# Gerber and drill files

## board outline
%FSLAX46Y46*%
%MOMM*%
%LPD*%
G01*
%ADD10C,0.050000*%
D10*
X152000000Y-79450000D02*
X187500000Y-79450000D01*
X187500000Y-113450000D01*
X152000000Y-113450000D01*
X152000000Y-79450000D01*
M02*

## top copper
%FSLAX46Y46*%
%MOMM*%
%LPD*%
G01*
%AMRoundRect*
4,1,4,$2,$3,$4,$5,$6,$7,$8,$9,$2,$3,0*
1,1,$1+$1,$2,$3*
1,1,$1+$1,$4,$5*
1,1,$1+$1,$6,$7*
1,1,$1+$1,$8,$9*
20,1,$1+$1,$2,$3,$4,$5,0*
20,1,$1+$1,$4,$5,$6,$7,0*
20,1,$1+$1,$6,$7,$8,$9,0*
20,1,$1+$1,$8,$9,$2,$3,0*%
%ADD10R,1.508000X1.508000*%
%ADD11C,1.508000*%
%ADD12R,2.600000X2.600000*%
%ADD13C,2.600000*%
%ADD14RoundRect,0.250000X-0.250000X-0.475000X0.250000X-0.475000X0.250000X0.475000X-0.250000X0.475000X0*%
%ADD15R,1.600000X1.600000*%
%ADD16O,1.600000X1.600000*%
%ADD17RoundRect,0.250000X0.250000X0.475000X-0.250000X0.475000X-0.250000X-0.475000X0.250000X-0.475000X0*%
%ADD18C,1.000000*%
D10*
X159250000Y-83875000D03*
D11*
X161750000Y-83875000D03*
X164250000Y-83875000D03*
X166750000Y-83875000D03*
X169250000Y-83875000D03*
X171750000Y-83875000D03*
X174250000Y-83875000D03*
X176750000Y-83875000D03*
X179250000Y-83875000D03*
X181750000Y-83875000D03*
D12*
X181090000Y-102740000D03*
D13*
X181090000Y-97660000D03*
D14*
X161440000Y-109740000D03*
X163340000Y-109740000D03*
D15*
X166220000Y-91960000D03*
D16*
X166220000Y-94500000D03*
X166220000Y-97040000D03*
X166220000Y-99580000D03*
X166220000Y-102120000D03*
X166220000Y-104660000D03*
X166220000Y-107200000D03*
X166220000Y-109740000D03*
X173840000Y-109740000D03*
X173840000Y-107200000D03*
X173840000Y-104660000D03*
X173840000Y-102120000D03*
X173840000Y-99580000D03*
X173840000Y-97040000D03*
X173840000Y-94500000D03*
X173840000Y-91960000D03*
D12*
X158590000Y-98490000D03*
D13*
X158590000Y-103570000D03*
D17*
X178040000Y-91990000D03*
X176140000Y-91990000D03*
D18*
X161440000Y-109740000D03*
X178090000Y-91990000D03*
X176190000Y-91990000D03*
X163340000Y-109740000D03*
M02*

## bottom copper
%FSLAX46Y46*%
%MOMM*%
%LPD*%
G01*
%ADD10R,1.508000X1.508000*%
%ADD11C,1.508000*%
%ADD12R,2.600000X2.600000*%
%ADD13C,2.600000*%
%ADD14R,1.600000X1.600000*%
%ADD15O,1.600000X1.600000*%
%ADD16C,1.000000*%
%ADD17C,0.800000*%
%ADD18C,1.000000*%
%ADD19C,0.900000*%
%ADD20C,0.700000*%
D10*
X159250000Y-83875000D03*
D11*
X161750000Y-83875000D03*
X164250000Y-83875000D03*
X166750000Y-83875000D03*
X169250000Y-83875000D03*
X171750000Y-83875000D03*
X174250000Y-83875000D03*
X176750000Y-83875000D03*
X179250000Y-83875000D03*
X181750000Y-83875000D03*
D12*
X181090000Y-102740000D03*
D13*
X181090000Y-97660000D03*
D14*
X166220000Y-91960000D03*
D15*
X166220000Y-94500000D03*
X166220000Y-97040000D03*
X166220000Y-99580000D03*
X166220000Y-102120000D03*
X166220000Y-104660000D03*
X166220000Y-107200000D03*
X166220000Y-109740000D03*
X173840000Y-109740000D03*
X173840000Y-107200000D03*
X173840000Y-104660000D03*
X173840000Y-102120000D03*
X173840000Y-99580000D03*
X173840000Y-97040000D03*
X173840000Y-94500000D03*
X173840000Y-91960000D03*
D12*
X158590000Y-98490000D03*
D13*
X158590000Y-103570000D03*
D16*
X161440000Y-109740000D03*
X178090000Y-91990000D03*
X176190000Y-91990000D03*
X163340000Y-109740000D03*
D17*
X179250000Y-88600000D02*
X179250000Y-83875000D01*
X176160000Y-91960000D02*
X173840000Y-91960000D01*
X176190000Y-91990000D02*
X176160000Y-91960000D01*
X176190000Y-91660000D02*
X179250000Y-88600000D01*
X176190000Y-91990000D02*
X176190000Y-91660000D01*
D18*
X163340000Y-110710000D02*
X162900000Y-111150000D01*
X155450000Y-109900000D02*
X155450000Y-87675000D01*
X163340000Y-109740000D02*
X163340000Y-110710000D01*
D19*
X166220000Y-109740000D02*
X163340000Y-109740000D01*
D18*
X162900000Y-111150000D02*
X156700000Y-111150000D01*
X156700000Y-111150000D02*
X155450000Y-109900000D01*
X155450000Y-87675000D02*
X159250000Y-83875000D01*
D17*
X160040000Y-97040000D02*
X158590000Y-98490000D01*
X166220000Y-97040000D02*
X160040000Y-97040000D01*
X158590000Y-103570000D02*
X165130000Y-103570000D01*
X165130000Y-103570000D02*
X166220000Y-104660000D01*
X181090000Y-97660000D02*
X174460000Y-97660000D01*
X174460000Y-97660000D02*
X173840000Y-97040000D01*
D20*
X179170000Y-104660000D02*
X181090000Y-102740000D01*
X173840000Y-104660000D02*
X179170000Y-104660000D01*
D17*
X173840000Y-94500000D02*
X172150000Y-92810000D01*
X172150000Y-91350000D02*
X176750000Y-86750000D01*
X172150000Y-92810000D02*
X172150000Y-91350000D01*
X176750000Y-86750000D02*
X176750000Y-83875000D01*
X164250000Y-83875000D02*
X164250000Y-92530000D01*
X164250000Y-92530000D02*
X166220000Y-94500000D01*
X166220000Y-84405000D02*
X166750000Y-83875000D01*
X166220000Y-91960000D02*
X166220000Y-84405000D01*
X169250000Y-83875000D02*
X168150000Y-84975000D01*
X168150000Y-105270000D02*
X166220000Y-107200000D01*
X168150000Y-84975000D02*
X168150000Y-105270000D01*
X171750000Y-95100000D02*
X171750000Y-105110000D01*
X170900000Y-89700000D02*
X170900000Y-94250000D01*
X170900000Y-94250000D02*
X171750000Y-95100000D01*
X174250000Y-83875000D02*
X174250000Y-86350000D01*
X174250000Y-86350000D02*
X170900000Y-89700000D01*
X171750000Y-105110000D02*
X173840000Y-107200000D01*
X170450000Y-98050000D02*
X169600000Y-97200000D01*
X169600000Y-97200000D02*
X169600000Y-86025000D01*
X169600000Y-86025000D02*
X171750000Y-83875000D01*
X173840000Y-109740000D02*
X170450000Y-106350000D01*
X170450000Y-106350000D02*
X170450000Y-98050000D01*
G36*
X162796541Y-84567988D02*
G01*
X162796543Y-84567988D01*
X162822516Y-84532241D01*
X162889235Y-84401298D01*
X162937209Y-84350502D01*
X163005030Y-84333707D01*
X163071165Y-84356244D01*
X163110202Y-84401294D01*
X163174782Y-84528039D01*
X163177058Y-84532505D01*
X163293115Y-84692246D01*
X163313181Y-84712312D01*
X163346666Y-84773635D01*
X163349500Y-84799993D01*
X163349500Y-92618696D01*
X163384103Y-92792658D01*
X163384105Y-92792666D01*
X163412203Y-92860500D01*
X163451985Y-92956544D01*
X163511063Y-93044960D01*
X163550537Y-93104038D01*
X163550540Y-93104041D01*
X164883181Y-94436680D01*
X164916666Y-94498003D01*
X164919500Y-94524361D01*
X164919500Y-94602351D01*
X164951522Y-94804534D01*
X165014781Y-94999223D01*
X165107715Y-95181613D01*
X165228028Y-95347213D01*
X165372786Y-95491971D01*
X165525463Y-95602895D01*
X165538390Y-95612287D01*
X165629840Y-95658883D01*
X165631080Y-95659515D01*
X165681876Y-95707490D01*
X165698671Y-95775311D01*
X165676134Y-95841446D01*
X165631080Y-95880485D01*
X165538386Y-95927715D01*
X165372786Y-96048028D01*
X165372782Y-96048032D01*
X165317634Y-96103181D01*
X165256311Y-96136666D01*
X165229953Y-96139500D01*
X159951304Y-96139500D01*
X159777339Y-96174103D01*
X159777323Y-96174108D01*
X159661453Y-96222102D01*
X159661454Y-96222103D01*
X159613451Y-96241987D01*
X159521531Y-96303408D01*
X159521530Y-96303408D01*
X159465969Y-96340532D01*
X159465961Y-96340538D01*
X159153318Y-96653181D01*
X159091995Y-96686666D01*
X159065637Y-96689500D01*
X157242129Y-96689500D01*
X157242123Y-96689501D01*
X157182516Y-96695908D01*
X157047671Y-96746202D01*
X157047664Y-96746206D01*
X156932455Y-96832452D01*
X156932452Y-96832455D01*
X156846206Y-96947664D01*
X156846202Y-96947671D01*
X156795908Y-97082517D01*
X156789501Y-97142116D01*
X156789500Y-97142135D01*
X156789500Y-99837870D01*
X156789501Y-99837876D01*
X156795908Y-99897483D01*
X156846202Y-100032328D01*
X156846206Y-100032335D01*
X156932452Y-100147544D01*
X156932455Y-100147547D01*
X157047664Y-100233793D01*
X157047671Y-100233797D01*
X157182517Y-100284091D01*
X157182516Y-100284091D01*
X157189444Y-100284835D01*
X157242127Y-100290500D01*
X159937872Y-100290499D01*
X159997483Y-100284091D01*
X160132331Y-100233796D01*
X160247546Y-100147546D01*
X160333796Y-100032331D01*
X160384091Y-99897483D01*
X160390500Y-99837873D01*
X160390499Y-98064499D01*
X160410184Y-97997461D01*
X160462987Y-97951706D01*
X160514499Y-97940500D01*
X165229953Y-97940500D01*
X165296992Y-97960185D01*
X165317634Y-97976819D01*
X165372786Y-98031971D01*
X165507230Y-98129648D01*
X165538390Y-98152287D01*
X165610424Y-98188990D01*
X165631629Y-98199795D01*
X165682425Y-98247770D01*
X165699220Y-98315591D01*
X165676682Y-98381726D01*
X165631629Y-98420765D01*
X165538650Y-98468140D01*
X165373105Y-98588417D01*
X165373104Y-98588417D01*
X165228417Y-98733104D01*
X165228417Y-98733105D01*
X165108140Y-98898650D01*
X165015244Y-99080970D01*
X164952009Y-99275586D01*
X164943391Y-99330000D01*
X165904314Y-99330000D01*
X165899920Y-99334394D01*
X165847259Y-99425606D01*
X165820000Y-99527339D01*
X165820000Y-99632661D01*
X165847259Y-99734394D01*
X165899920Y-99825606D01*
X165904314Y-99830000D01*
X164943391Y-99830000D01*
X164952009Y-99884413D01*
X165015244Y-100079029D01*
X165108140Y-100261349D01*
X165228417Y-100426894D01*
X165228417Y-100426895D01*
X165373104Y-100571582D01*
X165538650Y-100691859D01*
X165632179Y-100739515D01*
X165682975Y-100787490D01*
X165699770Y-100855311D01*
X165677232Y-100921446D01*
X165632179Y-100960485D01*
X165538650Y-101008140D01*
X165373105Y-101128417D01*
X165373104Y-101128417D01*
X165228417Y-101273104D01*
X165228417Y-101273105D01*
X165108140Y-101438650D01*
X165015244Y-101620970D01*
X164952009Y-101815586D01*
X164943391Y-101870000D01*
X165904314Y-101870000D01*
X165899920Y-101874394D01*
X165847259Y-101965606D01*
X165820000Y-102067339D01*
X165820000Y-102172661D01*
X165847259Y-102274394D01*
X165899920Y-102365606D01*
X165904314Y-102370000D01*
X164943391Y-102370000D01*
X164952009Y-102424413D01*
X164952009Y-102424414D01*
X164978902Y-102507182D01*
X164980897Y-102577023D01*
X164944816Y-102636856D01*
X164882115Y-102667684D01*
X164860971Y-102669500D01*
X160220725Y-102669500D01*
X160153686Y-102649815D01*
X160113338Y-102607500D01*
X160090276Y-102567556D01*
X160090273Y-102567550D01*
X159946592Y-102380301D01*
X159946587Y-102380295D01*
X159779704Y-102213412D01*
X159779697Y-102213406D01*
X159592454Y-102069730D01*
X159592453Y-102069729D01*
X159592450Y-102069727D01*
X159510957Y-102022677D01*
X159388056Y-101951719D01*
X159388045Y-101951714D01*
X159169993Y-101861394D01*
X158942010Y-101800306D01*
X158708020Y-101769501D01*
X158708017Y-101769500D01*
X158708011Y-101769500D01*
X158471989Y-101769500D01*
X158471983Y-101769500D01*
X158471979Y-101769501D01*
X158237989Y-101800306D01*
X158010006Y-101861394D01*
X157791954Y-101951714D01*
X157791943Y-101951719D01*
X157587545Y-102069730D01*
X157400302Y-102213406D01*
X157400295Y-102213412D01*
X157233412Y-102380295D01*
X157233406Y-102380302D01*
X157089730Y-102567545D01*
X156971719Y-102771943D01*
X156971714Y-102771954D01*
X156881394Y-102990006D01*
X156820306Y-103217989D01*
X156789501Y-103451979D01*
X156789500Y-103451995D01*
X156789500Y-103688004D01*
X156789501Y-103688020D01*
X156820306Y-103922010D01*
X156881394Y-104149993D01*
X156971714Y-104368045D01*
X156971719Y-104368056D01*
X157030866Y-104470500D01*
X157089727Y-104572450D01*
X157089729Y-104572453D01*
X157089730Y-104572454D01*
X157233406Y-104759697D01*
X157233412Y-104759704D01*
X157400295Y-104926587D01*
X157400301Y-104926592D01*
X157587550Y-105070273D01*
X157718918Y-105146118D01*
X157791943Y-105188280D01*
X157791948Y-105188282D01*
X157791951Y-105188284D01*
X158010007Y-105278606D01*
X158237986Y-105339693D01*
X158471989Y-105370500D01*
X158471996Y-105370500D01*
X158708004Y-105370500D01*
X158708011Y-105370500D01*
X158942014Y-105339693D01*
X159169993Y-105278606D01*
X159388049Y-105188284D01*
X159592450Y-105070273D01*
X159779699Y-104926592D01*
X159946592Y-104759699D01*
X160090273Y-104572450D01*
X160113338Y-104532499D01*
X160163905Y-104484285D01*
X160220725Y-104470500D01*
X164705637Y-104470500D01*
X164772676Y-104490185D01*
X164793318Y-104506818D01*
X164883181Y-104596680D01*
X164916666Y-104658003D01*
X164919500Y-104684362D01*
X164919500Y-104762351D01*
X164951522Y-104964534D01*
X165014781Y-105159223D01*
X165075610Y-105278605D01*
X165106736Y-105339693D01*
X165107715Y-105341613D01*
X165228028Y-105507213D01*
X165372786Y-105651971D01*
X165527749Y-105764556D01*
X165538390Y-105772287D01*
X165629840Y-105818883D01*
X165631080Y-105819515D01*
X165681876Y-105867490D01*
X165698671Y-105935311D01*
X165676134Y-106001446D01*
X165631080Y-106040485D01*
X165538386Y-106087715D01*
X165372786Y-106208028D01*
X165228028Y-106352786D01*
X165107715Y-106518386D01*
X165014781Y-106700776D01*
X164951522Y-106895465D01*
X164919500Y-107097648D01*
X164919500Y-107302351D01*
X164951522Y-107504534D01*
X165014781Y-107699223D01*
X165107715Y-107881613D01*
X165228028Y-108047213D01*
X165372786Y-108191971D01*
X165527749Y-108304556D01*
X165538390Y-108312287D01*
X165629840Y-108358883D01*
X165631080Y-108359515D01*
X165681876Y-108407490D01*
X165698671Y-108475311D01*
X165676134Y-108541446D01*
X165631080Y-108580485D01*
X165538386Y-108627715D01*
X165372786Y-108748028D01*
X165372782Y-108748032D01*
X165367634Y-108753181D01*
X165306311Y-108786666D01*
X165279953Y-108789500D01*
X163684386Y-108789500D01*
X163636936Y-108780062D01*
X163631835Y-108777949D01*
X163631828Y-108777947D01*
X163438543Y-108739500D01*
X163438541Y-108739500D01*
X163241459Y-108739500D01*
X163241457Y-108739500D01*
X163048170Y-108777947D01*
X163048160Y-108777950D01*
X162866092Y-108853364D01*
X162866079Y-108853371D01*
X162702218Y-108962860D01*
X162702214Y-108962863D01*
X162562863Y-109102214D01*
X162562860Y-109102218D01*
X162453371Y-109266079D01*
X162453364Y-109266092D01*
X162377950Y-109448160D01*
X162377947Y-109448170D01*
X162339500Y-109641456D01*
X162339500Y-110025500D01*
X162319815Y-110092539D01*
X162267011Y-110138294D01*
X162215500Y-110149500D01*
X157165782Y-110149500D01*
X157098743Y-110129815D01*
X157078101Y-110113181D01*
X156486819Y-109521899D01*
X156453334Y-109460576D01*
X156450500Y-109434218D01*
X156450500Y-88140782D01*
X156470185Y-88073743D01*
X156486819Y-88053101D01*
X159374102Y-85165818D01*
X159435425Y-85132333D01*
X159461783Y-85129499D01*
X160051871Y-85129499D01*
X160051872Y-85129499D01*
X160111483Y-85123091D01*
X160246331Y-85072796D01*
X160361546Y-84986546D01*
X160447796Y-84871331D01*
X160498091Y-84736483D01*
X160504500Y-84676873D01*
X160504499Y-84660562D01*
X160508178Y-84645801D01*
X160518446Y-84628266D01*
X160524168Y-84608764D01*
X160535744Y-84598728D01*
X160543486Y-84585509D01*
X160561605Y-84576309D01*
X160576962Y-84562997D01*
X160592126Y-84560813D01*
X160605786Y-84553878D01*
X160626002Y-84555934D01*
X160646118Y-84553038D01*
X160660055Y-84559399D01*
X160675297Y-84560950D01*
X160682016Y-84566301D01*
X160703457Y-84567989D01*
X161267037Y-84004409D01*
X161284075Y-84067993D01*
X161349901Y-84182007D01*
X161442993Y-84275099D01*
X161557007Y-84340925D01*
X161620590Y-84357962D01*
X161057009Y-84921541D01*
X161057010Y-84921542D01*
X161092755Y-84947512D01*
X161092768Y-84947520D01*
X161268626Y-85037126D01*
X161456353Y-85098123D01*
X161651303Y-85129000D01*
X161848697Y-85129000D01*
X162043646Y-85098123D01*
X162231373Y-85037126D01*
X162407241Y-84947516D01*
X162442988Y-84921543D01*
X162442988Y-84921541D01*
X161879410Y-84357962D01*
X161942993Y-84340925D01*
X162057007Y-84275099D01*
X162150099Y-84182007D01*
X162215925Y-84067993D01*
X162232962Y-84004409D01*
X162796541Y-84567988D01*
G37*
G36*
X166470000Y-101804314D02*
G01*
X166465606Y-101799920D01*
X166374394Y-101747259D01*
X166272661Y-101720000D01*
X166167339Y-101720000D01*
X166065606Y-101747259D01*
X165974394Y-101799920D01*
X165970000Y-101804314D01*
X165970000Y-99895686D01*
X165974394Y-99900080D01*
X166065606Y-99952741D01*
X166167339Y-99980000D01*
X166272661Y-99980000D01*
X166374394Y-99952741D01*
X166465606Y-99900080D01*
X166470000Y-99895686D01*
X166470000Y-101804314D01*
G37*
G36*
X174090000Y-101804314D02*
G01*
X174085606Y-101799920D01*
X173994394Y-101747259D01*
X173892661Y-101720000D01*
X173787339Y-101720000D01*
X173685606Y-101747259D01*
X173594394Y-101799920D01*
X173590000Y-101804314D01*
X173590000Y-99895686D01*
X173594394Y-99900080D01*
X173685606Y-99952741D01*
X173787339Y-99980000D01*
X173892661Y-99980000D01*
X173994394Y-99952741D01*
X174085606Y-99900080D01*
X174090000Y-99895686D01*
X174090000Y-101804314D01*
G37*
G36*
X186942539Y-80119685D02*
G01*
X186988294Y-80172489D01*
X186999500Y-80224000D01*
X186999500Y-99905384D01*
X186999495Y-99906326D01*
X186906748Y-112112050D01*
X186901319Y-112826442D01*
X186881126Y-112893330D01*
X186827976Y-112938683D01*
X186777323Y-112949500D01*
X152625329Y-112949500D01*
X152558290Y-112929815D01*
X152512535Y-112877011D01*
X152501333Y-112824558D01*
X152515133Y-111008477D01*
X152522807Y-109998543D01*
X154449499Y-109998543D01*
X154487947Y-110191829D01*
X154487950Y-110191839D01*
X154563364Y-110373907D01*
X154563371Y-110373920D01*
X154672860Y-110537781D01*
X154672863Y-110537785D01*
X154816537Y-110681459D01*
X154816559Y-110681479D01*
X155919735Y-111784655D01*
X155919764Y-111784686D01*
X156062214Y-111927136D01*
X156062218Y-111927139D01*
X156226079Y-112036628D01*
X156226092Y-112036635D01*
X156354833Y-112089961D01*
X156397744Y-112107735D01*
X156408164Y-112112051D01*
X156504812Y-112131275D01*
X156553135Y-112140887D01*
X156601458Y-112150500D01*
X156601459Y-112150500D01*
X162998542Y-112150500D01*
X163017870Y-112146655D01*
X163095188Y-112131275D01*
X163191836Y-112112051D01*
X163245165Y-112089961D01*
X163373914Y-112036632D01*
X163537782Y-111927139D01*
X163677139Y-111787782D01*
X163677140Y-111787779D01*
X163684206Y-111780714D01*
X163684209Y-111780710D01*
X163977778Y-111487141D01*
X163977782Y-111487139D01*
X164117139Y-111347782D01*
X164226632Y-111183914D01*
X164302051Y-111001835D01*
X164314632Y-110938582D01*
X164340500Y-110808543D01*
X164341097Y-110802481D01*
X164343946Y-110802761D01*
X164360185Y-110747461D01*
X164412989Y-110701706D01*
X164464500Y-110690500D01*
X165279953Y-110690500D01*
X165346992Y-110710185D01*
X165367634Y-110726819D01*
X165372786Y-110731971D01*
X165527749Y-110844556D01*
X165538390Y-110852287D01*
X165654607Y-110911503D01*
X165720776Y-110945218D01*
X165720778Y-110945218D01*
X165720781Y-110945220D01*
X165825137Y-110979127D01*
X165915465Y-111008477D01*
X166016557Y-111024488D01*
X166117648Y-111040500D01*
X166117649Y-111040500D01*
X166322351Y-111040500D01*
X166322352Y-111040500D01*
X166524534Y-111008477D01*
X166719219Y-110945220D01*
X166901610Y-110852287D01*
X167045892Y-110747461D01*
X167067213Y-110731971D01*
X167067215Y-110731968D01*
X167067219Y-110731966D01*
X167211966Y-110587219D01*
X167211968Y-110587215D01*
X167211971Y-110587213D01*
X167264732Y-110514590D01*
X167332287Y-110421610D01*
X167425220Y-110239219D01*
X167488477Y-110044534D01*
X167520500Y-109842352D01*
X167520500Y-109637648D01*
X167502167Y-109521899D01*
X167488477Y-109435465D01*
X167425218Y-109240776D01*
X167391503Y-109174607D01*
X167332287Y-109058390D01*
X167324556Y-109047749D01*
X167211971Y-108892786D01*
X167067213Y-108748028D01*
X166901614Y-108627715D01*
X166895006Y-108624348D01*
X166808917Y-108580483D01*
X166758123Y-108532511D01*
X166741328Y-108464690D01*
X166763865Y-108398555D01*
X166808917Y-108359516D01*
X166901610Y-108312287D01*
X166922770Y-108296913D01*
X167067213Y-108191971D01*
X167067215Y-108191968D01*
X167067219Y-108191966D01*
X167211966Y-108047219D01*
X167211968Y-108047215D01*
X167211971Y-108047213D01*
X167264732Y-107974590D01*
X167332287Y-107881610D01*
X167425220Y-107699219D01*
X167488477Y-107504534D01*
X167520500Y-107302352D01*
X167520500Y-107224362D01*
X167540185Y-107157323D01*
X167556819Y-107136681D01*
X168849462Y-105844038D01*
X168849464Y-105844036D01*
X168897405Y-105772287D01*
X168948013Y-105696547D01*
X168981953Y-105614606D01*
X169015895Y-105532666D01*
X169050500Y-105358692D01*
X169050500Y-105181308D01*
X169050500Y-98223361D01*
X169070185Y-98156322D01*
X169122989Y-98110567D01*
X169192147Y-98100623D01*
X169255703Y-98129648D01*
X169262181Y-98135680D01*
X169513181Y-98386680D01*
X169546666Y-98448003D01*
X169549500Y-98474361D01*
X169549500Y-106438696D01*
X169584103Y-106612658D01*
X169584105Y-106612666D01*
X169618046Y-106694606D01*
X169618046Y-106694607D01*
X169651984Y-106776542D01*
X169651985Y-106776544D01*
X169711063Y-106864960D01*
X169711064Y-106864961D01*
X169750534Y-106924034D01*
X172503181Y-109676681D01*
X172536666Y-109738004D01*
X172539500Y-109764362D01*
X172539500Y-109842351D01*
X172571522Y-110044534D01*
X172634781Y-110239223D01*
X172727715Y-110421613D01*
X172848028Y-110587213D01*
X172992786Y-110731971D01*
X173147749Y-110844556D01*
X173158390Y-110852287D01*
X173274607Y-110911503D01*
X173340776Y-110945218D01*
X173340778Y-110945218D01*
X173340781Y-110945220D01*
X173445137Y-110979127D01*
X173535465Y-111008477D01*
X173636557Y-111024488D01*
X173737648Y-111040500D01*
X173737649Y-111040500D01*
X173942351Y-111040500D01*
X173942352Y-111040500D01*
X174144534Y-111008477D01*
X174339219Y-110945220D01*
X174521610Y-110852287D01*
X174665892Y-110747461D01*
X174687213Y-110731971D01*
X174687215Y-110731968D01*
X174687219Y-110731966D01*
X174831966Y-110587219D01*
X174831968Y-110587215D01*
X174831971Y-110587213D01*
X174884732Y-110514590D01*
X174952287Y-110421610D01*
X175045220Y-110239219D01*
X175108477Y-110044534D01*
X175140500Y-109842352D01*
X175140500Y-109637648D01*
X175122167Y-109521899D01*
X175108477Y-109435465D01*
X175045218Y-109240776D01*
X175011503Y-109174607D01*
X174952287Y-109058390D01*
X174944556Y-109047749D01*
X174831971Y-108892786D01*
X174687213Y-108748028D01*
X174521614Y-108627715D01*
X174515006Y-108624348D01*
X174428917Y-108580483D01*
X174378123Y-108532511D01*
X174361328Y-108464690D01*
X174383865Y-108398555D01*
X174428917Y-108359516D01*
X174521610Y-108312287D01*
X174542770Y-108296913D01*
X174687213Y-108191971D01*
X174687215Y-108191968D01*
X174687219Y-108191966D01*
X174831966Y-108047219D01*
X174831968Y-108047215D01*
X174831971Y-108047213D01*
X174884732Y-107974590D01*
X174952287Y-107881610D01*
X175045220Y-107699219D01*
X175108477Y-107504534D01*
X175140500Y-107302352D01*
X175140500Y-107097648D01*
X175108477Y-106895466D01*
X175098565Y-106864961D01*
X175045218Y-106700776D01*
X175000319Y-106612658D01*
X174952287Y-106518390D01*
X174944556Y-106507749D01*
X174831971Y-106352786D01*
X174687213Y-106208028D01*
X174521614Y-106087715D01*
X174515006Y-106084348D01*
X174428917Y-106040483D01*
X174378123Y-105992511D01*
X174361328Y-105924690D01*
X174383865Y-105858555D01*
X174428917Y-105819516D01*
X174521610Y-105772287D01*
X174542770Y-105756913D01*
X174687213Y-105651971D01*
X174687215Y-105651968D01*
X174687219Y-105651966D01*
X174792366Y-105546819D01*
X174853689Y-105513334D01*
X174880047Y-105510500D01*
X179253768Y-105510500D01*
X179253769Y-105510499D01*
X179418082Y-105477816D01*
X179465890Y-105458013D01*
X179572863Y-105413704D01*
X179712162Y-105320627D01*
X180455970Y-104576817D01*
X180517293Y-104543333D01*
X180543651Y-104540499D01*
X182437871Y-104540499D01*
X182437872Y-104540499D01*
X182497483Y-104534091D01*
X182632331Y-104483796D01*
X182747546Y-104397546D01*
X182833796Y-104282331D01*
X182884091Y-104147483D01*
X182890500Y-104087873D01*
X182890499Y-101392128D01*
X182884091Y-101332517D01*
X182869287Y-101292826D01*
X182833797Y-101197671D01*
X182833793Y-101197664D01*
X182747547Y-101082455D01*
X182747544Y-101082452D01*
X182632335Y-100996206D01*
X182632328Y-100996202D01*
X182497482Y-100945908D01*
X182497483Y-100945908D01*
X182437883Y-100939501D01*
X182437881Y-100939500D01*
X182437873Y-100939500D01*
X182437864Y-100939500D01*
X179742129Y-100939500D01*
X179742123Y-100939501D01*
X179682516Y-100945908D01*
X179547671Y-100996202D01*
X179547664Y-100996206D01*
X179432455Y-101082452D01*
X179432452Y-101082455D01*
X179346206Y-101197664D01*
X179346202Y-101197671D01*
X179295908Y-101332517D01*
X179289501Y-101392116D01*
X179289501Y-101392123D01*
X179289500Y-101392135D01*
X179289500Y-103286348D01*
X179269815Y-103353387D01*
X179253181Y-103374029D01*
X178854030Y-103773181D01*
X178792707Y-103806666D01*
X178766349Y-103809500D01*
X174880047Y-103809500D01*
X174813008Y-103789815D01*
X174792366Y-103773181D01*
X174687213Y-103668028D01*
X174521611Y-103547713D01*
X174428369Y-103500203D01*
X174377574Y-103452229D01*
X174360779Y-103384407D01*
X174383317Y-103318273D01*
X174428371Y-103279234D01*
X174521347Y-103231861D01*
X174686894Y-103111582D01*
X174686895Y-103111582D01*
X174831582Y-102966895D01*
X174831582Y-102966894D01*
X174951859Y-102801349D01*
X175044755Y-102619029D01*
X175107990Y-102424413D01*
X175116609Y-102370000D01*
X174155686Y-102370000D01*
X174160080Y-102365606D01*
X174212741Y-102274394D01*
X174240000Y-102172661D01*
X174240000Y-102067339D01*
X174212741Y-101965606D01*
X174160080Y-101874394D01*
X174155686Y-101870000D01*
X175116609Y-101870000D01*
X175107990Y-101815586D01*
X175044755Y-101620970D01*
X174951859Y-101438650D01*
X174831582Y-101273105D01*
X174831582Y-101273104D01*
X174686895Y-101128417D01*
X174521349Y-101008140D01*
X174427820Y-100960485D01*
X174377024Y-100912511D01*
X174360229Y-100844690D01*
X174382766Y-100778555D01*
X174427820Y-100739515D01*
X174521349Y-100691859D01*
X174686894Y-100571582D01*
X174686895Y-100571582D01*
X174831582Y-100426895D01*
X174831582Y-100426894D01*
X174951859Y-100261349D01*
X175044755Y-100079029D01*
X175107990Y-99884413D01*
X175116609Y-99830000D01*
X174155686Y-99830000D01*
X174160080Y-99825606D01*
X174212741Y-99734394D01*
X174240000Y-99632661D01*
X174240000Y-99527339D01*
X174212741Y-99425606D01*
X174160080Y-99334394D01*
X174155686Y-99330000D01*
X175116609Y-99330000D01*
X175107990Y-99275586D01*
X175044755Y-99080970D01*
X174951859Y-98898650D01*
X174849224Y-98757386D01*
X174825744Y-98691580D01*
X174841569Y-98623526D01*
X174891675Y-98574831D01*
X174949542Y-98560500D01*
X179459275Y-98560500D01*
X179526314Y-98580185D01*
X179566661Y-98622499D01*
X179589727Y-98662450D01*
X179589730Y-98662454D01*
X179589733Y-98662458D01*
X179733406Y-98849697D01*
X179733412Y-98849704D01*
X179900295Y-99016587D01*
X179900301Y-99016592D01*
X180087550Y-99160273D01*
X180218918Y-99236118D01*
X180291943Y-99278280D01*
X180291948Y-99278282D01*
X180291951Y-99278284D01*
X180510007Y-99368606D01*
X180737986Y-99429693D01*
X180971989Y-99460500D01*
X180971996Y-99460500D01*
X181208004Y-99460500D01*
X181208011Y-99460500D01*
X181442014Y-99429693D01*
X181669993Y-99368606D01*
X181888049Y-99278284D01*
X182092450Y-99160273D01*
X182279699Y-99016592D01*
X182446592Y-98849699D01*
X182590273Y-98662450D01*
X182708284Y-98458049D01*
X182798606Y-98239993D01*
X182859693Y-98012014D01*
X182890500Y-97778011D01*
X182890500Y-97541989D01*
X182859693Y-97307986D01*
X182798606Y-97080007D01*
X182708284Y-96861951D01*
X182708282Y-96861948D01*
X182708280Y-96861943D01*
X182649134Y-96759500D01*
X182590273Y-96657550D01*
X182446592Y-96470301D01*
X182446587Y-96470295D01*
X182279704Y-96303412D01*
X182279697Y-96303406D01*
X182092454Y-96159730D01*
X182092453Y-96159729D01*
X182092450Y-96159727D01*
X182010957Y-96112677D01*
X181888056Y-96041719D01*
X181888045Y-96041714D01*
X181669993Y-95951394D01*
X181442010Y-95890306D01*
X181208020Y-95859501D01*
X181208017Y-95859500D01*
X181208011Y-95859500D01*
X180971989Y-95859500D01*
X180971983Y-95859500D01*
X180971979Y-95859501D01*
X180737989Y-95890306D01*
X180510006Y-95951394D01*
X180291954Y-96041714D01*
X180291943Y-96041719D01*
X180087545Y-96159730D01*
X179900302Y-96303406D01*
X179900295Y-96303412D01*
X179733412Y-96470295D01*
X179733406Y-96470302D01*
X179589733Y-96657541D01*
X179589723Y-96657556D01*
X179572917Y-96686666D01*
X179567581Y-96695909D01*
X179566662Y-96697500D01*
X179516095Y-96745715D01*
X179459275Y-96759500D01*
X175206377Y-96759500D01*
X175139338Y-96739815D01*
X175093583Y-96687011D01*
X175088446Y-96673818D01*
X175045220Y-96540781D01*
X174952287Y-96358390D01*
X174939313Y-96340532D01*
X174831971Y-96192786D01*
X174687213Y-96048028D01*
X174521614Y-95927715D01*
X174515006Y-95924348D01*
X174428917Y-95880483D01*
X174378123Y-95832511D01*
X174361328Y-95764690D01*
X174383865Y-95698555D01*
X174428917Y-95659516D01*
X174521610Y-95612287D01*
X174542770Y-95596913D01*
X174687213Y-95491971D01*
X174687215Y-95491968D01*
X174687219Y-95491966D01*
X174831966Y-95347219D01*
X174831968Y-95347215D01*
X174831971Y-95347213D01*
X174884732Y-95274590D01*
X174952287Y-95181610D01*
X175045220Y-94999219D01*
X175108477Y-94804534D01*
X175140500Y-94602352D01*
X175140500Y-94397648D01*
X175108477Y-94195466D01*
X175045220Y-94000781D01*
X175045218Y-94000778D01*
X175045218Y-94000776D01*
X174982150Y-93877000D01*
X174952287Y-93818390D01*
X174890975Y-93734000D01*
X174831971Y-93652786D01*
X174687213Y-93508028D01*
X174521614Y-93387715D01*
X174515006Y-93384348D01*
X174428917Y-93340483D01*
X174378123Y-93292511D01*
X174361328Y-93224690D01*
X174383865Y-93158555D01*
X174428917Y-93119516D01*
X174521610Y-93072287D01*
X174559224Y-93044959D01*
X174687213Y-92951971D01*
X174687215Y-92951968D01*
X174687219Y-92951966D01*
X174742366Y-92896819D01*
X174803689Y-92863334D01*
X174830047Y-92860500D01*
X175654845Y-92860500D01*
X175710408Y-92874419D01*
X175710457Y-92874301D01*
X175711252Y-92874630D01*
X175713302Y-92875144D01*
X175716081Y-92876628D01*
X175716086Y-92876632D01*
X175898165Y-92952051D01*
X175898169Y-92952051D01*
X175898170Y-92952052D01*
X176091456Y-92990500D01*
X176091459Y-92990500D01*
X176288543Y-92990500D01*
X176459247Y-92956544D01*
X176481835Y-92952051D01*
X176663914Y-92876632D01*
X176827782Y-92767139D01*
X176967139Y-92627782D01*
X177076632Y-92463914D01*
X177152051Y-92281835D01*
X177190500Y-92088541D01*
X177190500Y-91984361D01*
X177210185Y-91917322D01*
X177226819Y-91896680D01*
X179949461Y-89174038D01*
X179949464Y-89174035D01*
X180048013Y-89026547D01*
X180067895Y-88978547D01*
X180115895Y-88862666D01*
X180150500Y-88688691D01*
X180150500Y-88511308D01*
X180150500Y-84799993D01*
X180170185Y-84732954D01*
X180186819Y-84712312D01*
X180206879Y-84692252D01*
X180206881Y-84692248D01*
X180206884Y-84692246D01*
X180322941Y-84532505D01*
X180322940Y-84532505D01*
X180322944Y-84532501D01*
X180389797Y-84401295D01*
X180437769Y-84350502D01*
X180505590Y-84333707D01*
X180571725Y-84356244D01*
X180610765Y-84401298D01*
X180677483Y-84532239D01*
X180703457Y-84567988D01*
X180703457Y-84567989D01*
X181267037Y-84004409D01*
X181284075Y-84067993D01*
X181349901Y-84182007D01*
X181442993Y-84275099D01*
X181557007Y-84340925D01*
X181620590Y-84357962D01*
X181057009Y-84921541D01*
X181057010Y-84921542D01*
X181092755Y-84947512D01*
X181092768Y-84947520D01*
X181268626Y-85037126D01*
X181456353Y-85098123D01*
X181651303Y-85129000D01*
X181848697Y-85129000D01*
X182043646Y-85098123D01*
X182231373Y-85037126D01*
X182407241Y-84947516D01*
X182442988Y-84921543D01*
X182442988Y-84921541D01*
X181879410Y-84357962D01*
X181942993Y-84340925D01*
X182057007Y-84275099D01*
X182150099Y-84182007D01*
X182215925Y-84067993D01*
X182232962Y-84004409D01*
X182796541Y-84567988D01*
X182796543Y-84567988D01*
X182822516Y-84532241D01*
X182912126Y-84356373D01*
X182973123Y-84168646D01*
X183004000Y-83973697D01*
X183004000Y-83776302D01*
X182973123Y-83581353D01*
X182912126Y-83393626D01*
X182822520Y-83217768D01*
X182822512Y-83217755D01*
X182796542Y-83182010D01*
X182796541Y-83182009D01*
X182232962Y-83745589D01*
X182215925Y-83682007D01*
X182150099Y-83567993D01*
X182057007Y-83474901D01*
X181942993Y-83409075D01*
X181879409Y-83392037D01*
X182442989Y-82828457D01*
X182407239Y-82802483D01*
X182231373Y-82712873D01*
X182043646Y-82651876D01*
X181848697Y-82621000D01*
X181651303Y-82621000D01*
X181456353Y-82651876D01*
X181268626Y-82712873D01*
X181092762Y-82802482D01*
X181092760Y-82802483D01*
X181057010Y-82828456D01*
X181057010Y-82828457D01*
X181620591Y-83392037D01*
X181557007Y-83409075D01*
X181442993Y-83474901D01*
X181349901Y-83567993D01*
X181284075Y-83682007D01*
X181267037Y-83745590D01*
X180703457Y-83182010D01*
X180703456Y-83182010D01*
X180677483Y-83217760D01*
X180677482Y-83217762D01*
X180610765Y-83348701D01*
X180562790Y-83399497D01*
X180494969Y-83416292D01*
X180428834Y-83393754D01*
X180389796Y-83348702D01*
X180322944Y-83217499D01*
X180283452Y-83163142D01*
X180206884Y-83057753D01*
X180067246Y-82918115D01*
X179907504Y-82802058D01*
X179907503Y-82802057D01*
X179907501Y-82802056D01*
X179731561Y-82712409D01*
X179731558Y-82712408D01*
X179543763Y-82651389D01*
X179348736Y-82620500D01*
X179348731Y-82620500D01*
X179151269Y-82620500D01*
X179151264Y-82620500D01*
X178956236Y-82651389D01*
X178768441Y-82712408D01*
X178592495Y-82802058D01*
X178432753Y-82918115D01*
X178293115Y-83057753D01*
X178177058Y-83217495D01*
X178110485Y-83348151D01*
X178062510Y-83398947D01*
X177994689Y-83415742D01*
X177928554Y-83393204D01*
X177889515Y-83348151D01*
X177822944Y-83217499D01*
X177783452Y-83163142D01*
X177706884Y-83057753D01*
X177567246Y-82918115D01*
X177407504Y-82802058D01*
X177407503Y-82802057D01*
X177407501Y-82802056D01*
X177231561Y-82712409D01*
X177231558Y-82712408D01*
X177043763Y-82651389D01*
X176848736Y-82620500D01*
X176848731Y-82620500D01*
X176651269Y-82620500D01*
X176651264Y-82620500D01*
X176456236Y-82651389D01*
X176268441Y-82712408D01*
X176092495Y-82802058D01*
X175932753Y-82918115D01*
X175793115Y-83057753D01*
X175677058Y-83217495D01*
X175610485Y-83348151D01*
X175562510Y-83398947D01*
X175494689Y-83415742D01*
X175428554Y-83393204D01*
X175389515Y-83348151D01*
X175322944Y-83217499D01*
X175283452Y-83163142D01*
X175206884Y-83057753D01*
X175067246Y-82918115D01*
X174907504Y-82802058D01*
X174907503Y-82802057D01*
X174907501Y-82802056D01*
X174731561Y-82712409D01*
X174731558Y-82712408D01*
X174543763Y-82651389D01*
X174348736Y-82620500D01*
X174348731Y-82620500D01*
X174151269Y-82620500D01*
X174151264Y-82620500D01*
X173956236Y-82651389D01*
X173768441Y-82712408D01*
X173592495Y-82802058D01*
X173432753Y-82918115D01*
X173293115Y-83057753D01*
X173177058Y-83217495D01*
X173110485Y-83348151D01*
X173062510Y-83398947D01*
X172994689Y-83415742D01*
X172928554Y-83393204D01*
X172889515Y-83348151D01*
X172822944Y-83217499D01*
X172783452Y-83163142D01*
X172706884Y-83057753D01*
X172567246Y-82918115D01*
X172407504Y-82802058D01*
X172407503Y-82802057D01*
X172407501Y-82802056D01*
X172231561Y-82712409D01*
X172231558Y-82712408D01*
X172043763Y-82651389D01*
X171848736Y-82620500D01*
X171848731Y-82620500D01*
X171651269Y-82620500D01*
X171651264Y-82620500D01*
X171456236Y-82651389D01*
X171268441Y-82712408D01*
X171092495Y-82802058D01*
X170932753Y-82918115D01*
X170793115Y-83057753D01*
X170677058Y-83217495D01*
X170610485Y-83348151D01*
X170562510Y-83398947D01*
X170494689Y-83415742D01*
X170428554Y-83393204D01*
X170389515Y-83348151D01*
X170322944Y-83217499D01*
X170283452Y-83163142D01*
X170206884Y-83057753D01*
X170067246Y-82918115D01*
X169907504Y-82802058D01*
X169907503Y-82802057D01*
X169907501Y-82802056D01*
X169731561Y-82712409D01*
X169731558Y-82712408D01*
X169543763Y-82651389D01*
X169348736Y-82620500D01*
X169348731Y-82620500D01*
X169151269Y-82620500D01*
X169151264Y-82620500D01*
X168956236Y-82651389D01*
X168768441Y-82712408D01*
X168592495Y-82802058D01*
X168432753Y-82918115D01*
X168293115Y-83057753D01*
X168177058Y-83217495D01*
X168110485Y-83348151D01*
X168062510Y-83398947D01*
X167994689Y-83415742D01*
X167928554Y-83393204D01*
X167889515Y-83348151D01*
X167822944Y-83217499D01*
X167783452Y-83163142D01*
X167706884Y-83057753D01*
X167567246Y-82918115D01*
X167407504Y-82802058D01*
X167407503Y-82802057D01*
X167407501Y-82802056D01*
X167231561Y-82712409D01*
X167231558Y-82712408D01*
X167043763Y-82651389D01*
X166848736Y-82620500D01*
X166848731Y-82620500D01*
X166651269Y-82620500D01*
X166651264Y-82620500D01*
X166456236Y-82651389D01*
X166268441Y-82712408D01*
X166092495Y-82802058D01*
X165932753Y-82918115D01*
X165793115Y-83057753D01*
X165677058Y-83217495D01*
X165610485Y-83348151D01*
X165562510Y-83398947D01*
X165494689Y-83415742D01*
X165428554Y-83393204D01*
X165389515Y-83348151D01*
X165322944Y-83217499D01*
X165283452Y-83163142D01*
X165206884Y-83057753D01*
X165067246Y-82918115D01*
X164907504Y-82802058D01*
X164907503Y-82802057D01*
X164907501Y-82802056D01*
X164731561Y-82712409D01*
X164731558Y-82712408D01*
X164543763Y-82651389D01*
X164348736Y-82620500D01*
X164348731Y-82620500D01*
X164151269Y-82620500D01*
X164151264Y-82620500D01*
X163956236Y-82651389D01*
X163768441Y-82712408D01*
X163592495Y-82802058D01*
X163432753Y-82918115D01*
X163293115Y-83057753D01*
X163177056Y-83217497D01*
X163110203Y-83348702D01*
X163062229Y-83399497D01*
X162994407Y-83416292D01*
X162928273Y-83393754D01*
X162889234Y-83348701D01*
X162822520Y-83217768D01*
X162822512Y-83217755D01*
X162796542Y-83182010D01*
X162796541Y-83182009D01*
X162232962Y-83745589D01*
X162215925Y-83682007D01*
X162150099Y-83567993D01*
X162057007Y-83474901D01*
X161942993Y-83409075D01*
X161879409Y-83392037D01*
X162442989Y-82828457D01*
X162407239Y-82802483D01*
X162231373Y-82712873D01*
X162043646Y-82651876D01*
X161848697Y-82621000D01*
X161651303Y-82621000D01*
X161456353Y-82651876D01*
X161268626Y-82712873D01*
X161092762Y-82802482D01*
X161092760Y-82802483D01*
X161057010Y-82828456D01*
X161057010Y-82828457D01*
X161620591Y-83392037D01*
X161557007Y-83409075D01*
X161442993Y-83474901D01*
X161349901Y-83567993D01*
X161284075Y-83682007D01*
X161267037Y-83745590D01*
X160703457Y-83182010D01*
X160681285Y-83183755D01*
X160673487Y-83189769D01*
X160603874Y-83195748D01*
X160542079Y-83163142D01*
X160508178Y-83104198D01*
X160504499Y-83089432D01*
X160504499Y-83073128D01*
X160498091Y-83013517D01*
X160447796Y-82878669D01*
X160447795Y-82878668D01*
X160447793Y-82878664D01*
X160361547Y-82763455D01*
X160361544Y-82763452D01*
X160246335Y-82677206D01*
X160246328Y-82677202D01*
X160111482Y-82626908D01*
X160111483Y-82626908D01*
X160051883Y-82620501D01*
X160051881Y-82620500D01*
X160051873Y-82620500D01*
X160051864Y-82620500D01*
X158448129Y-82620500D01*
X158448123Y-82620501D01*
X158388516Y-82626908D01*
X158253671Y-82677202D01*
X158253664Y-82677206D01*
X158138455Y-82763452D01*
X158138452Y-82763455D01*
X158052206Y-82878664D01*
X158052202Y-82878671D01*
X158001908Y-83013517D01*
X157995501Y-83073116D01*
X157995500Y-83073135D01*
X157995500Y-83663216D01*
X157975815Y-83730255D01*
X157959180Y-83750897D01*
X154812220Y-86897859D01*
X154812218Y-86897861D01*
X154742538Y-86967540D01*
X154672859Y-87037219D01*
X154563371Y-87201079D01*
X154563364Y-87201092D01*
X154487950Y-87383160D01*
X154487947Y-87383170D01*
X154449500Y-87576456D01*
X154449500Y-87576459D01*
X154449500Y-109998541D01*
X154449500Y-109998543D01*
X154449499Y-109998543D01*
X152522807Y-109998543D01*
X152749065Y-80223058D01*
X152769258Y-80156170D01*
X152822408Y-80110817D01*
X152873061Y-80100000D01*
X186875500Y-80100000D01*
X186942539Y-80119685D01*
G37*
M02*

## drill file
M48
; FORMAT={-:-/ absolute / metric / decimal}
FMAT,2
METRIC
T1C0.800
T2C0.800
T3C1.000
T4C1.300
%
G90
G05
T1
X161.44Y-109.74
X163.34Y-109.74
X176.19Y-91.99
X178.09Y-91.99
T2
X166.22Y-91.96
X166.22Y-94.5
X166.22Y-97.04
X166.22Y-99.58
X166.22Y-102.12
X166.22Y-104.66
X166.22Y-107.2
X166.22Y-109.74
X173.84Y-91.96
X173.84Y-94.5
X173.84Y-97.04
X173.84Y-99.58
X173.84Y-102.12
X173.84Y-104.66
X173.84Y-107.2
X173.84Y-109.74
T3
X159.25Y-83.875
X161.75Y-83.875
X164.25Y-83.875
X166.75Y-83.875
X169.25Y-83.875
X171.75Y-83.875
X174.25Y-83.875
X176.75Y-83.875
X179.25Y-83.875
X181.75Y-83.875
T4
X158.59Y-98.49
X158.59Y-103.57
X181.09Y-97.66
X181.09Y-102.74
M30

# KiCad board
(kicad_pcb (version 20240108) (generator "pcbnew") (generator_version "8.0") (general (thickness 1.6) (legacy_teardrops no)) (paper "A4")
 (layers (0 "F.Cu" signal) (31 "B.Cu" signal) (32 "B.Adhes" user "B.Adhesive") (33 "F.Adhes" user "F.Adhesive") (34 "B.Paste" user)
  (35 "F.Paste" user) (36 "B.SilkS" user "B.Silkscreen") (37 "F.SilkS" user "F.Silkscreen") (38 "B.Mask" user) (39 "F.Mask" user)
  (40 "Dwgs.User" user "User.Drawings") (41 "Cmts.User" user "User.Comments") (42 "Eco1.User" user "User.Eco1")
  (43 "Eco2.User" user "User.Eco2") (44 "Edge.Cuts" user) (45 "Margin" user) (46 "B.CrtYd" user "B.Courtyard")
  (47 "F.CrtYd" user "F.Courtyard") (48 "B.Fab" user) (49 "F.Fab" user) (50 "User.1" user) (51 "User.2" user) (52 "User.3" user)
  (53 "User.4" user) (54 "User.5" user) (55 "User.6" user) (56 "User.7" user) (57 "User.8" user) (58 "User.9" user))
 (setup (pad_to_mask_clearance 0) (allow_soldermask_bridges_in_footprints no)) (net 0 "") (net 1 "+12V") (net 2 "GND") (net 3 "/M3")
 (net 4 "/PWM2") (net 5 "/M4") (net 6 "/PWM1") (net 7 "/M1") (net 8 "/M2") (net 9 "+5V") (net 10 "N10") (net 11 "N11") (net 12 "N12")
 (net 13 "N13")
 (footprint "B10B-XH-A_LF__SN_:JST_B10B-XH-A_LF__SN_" (layer "F.Cu") (at 170.5 84.4 180)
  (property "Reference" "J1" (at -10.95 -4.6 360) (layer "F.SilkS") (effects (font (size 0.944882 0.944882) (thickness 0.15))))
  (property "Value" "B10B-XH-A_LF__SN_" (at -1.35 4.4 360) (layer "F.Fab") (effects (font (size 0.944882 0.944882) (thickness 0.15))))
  (pad "1" thru_hole rect (at 11.25 0.525 180) (size 1.508 1.508) (drill 1) (layers "*.Cu" "*.Mask") (remove_unused_layers no)
   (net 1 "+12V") (solder_mask_margin 0.102))
  (pad "2" thru_hole circle (at 8.75 0.525 180) (size 1.508 1.508) (drill 1) (layers "*.Cu" "*.Mask") (remove_unused_layers no)
   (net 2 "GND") (solder_mask_margin 0.102))
  (pad "3" thru_hole circle (at 6.25 0.525 180) (size 1.508 1.508) (drill 1) (layers "*.Cu" "*.Mask") (remove_unused_layers no)
   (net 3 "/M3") (solder_mask_margin 0.102))
  (pad "4" thru_hole circle (at 3.75 0.525 180) (size 1.508 1.508) (drill 1) (layers "*.Cu" "*.Mask") (remove_unused_layers no)
   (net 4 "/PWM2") (solder_mask_margin 0.102))
  (pad "5" thru_hole circle (at 1.25 0.525 180) (size 1.508 1.508) (drill 1) (layers "*.Cu" "*.Mask") (remove_unused_layers no)
   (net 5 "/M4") (solder_mask_margin 0.102))
  (pad "6" thru_hole circle (at -1.25 0.525 180) (size 1.508 1.508) (drill 1) (layers "*.Cu" "*.Mask") (remove_unused_layers no)
   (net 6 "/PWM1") (solder_mask_margin 0.102))
  (pad "7" thru_hole circle (at -3.75 0.525 180) (size 1.508 1.508) (drill 1) (layers "*.Cu" "*.Mask") (remove_unused_layers no)
   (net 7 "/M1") (solder_mask_margin 0.102))
  (pad "8" thru_hole circle (at -6.25 0.525 180) (size 1.508 1.508) (drill 1) (layers "*.Cu" "*.Mask") (remove_unused_layers no)
   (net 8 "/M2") (solder_mask_margin 0.102))
  (pad "9" thru_hole circle (at -8.75 0.525 180) (size 1.508 1.508) (drill 1) (layers "*.Cu" "*.Mask") (remove_unused_layers no)
   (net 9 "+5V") (solder_mask_margin 0.102))
  (pad "10" thru_hole circle (at -11.25 0.525 180) (size 1.508 1.508) (drill 1) (layers "*.Cu" "*.Mask") (remove_unused_layers no)
   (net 2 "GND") (solder_mask_margin 0.102)))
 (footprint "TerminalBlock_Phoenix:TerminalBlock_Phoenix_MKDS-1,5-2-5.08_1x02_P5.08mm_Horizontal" (layer "F.Cu") (at 181.09 102.74 90)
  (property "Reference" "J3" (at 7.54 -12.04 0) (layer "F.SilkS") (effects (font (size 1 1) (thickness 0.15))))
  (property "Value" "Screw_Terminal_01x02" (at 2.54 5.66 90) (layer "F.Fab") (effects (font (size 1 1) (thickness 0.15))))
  (pad "1" thru_hole rect (at 0 0 90) (size 2.6 2.6) (drill 1.3) (layers "*.Cu" "*.Mask") (remove_unused_layers no) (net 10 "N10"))
  (pad "2" thru_hole circle (at 5.08 0 90) (size 2.6 2.6) (drill 1.3) (layers "*.Cu" "*.Mask") (remove_unused_layers no) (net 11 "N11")))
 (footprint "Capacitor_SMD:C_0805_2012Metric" (layer "F.Cu") (at 162.39 109.74)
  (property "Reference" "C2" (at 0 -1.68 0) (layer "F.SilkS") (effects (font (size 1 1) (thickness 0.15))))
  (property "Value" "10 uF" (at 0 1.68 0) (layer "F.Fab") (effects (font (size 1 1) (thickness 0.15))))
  (pad "1" smd roundrect (at -0.95 0) (size 1 1.45) (layers "F.Cu" "F.Paste" "F.Mask") (roundrect_rratio 0.25) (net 2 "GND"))
  (pad "2" smd roundrect (at 0.95 0) (size 1 1.45) (layers "F.Cu" "F.Paste" "F.Mask") (roundrect_rratio 0.25) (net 1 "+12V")))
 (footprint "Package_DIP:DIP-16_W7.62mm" (layer "F.Cu") (at 166.22 91.96)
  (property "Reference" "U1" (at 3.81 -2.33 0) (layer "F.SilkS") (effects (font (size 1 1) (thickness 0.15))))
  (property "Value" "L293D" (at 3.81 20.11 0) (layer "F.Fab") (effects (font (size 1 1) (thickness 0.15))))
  (pad "1" thru_hole rect (at 0 0) (size 1.6 1.6) (drill 0.8) (layers "*.Cu" "*.Mask") (remove_unused_layers no) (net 4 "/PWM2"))
  (pad "2" thru_hole oval (at 0 2.54) (size 1.6 1.6) (drill 0.8) (layers "*.Cu" "*.Mask") (remove_unused_layers no) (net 3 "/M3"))
  (pad "3" thru_hole oval (at 0 5.08) (size 1.6 1.6) (drill 0.8) (layers "*.Cu" "*.Mask") (remove_unused_layers no) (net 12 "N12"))
  (pad "4" thru_hole oval (at 0 7.62) (size 1.6 1.6) (drill 0.8) (layers "*.Cu" "*.Mask") (remove_unused_layers no) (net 2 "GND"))
  (pad "5" thru_hole oval (at 0 10.16) (size 1.6 1.6) (drill 0.8) (layers "*.Cu" "*.Mask") (remove_unused_layers no) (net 2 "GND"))
  (pad "6" thru_hole oval (at 0 12.7) (size 1.6 1.6) (drill 0.8) (layers "*.Cu" "*.Mask") (remove_unused_layers no) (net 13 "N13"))
  (pad "7" thru_hole oval (at 0 15.24) (size 1.6 1.6) (drill 0.8) (layers "*.Cu" "*.Mask") (remove_unused_layers no) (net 5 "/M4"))
  (pad "8" thru_hole oval (at 0 17.78) (size 1.6 1.6) (drill 0.8) (layers "*.Cu" "*.Mask") (remove_unused_layers no) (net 1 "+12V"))
  (pad "9" thru_hole oval (at 7.62 17.78) (size 1.6 1.6) (drill 0.8) (layers "*.Cu" "*.Mask") (remove_unused_layers no) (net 6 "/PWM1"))
  (pad "10" thru_hole oval (at 7.62 15.24) (size 1.6 1.6) (drill 0.8) (layers "*.Cu" "*.Mask") (remove_unused_layers no) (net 7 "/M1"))
  (pad "11" thru_hole oval (at 7.62 12.7) (size 1.6 1.6) (drill 0.8) (layers "*.Cu" "*.Mask") (remove_unused_layers no) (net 10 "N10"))
  (pad "12" thru_hole oval (at 7.62 10.16) (size 1.6 1.6) (drill 0.8) (layers "*.Cu" "*.Mask") (remove_unused_layers no) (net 2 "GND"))
  (pad "13" thru_hole oval (at 7.62 7.62) (size 1.6 1.6) (drill 0.8) (layers "*.Cu" "*.Mask") (remove_unused_layers no) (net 2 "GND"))
  (pad "14" thru_hole oval (at 7.62 5.08) (size 1.6 1.6) (drill 0.8) (layers "*.Cu" "*.Mask") (remove_unused_layers no) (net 11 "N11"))
  (pad "15" thru_hole oval (at 7.62 2.54) (size 1.6 1.6) (drill 0.8) (layers "*.Cu" "*.Mask") (remove_unused_layers no) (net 8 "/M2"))
  (pad "16" thru_hole oval (at 7.62 0) (size 1.6 1.6) (drill 0.8) (layers "*.Cu" "*.Mask") (remove_unused_layers no) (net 9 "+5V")))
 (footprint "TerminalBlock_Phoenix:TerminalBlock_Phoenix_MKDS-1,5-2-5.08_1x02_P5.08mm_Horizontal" (layer "F.Cu") (at 158.59 98.49 -90)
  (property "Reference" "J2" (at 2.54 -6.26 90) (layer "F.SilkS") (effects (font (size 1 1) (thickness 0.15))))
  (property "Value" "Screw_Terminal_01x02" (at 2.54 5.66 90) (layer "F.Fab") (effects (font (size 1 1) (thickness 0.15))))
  (pad "1" thru_hole rect (at 0 0 270) (size 2.6 2.6) (drill 1.3) (layers "*.Cu" "*.Mask") (remove_unused_layers no) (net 12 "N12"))
  (pad "2" thru_hole circle (at 5.08 0 270) (size 2.6 2.6) (drill 1.3) (layers "*.Cu" "*.Mask") (remove_unused_layers no) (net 13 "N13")))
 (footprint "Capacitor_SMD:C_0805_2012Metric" (layer "F.Cu") (at 177.09 91.99 180)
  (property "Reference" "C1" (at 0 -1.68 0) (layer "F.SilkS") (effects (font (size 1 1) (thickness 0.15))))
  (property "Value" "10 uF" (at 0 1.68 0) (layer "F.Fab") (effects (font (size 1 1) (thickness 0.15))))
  (pad "1" smd roundrect (at -0.95 0 180) (size 1 1.45) (layers "F.Cu" "F.Paste" "F.Mask") (roundrect_rratio 0.25) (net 2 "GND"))
  (pad "2" smd roundrect (at 0.95 0 180) (size 1 1.45) (layers "F.Cu" "F.Paste" "F.Mask") (roundrect_rratio 0.25) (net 9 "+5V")))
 (gr_rect (start 152 79.45) (end 187.5 113.45) (stroke (width 0.05) (type default)) (fill none) (layer "Edge.Cuts"))
 (via (at 161.44 109.74) (size 1) (drill 0.8) (layers "F.Cu" "B.Cu") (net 2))
 (via (at 178.09 91.99) (size 1) (drill 0.8) (layers "F.Cu" "B.Cu") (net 2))
 (via (at 176.19 91.99) (size 1) (drill 0.8) (layers "F.Cu" "B.Cu") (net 9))
 (segment (start 179.25 88.6) (end 179.25 83.875) (width 0.8) (layer "B.Cu") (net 9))
 (segment (start 176.16 91.96) (end 173.84 91.96) (width 0.8) (layer "B.Cu") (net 9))
 (segment (start 176.19 91.99) (end 176.16 91.96) (width 0.8) (layer "B.Cu") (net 9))
 (segment (start 176.19 91.66) (end 179.25 88.6) (width 0.8) (layer "B.Cu") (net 9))
 (segment (start 176.19 91.99) (end 176.19 91.66) (width 0.8) (layer "B.Cu") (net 9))
 (via (at 163.34 109.74) (size 1) (drill 0.8) (layers "F.Cu" "B.Cu") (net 1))
 (segment (start 163.34 110.71) (end 162.9 111.15) (width 1) (layer "B.Cu") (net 1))
 (segment (start 155.45 109.9) (end 155.45 87.675) (width 1) (layer "B.Cu") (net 1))
 (segment (start 163.34 109.74) (end 163.34 110.71) (width 1) (layer "B.Cu") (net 1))
 (segment (start 166.22 109.74) (end 163.34 109.74) (width 0.9) (layer "B.Cu") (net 1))
 (segment (start 162.9 111.15) (end 156.7 111.15) (width 1) (layer "B.Cu") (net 1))
 (segment (start 156.7 111.15) (end 155.45 109.9) (width 1) (layer "B.Cu") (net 1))
 (segment (start 155.45 87.675) (end 159.25 83.875) (width 1) (layer "B.Cu") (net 1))
 (segment (start 160.04 97.04) (end 158.59 98.49) (width 0.8) (layer "B.Cu") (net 12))
 (segment (start 166.22 97.04) (end 160.04 97.04) (width 0.8) (layer "B.Cu") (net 12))
 (segment (start 158.59 103.57) (end 165.13 103.57) (width 0.8) (layer "B.Cu") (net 13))
 (segment (start 165.13 103.57) (end 166.22 104.66) (width 0.8) (layer "B.Cu") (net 13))
 (segment (start 181.09 97.66) (end 174.46 97.66) (width 0.8) (layer "B.Cu") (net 11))
 (segment (start 174.46 97.66) (end 173.84 97.04) (width 0.8) (layer "B.Cu") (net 11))
 (segment (start 179.17 104.66) (end 181.09 102.74) (width 0.7) (layer "B.Cu") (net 10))
 (segment (start 173.84 104.66) (end 179.17 104.66) (width 0.7) (layer "B.Cu") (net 10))
 (segment (start 173.84 94.5) (end 172.15 92.81) (width 0.8) (layer "B.Cu") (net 8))
 (segment (start 172.15 91.35) (end 176.75 86.75) (width 0.8) (layer "B.Cu") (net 8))
 (segment (start 172.15 92.81) (end 172.15 91.35) (width 0.8) (layer "B.Cu") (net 8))
 (segment (start 176.75 86.75) (end 176.75 83.875) (width 0.8) (layer "B.Cu") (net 8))
 (segment (start 164.25 83.875) (end 164.25 92.53) (width 0.8) (layer "B.Cu") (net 3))
 (segment (start 164.25 92.53) (end 166.22 94.5) (width 0.8) (layer "B.Cu") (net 3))
 (segment (start 166.22 84.405) (end 166.75 83.875) (width 0.8) (layer "B.Cu") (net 4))
 (segment (start 166.22 91.96) (end 166.22 84.405) (width 0.8) (layer "B.Cu") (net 4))
 (segment (start 169.25 83.875) (end 168.15 84.975) (width 0.8) (layer "B.Cu") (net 5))
 (segment (start 168.15 105.27) (end 166.22 107.2) (width 0.8) (layer "B.Cu") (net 5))
 (segment (start 168.15 84.975) (end 168.15 105.27) (width 0.8) (layer "B.Cu") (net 5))
 (segment (start 171.75 95.1) (end 171.75 105.11) (width 0.8) (layer "B.Cu") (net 7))
 (segment (start 170.9 89.7) (end 170.9 94.25) (width 0.8) (layer "B.Cu") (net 7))
 (segment (start 170.9 94.25) (end 171.75 95.1) (width 0.8) (layer "B.Cu") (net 7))
 (segment (start 174.25 83.875) (end 174.25 86.35) (width 0.8) (layer "B.Cu") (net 7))
 (segment (start 174.25 86.35) (end 170.9 89.7) (width 0.8) (layer "B.Cu") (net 7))
 (segment (start 171.75 105.11) (end 173.84 107.2) (width 0.8) (layer "B.Cu") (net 7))
 (segment (start 170.45 98.05) (end 169.6 97.2) (width 0.8) (layer "B.Cu") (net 6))
 (segment (start 169.6 97.2) (end 169.6 86.025) (width 0.8) (layer "B.Cu") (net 6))
 (segment (start 169.6 86.025) (end 171.75 83.875) (width 0.8) (layer "B.Cu") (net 6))
 (segment (start 173.84 109.74) (end 170.45 106.35) (width 0.8) (layer "B.Cu") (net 6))
 (segment (start 170.45 106.35) (end 170.45 98.05) (width 0.8) (layer "B.Cu") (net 6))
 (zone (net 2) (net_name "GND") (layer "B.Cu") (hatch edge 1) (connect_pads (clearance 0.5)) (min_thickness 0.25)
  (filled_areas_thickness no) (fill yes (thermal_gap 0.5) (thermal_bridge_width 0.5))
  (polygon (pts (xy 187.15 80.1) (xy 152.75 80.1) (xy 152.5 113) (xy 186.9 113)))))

